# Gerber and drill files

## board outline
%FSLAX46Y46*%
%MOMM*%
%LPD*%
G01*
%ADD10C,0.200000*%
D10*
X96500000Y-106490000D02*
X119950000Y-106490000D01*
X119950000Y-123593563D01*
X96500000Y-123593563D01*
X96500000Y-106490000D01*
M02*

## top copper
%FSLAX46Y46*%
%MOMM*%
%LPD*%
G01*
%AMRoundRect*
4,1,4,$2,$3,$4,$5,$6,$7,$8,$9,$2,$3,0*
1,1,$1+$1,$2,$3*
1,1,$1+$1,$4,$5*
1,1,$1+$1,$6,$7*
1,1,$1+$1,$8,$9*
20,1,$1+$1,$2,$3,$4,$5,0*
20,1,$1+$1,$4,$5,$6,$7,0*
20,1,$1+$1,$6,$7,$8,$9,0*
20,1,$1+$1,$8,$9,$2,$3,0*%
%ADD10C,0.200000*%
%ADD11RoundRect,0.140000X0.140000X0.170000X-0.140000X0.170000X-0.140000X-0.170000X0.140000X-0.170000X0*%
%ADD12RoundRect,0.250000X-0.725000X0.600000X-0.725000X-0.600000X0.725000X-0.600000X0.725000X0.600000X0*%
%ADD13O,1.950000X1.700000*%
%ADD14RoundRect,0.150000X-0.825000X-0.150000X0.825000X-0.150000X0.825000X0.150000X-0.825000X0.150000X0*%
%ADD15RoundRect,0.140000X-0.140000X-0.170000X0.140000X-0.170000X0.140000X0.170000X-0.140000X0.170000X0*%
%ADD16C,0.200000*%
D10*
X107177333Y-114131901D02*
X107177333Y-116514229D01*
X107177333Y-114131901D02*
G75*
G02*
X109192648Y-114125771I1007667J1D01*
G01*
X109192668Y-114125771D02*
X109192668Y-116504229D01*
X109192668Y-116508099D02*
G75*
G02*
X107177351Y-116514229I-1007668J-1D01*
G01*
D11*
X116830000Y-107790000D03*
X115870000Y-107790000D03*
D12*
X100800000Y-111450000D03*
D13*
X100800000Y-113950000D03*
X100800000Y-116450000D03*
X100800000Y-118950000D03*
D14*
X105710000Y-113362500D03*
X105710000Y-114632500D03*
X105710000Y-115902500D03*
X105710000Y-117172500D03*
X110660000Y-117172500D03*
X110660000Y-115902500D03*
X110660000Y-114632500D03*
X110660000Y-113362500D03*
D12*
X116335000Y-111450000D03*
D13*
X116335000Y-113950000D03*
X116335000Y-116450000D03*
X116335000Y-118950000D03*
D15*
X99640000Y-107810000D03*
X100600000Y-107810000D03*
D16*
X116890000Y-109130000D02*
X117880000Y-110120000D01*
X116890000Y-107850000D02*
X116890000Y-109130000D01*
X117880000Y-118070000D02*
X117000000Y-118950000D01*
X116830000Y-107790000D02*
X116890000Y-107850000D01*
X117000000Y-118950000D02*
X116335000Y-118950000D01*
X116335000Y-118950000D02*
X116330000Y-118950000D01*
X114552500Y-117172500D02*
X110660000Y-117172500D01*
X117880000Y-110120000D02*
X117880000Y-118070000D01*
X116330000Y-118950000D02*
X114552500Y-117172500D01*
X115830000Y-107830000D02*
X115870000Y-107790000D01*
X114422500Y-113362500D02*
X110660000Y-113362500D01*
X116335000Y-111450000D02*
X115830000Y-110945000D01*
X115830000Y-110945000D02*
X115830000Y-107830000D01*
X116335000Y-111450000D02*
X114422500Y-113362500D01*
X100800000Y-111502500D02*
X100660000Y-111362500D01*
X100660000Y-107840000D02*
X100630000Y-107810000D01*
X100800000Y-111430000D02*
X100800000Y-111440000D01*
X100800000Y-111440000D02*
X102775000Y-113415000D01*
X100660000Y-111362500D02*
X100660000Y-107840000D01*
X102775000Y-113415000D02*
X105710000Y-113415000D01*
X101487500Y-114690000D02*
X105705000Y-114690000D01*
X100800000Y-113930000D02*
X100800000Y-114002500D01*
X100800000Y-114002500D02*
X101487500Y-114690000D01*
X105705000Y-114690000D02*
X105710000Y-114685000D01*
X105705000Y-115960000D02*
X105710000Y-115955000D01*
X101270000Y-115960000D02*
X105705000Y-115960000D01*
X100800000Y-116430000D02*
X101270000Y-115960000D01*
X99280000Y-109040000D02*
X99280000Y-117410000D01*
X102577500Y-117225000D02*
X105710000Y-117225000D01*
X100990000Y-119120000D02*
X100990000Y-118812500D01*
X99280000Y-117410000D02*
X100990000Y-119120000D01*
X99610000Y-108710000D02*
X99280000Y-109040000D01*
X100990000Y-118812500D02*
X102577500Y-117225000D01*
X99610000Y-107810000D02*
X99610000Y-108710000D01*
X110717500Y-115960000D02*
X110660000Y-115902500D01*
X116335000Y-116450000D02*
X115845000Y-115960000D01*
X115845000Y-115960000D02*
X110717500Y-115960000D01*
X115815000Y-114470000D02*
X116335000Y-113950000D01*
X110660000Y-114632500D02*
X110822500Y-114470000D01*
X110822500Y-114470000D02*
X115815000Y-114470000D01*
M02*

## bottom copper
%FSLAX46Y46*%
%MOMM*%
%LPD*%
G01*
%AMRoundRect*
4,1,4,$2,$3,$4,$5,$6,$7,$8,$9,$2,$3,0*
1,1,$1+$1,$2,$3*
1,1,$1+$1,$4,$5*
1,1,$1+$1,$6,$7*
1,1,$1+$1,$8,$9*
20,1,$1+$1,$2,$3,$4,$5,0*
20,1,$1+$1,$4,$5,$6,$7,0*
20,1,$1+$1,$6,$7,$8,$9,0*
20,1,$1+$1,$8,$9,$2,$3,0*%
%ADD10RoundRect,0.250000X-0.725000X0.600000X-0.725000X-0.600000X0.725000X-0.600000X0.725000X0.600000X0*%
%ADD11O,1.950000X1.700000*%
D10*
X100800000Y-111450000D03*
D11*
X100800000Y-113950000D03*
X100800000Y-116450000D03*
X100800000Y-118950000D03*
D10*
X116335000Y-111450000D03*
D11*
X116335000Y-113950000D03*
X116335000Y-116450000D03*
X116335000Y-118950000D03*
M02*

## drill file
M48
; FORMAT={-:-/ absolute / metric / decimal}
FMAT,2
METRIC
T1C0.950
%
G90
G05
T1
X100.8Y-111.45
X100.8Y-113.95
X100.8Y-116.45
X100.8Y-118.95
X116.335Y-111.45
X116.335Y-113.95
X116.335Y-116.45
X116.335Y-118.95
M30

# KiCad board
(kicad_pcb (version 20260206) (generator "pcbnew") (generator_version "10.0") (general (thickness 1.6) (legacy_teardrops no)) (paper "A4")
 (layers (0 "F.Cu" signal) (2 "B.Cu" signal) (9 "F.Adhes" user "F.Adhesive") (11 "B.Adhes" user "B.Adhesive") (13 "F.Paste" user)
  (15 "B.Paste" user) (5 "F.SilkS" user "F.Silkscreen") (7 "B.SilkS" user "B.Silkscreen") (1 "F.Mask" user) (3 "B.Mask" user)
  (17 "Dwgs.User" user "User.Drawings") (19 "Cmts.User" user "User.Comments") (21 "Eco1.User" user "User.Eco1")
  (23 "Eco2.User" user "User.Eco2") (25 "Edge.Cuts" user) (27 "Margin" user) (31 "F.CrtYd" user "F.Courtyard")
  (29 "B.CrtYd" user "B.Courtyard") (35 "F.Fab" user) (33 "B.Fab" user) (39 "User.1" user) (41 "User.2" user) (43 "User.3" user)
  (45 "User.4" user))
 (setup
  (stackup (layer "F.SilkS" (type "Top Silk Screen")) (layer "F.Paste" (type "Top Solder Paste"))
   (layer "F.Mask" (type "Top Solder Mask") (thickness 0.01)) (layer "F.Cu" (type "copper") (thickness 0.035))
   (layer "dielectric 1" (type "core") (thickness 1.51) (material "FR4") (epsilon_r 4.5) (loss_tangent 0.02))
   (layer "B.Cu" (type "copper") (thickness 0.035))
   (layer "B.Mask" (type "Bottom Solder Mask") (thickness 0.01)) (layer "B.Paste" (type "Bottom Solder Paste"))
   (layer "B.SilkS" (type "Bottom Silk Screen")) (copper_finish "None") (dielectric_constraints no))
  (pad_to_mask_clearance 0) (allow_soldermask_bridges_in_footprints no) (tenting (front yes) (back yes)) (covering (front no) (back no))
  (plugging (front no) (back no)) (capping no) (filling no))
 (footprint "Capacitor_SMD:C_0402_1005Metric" (layer "F.Cu") (at 116.35 107.79 180)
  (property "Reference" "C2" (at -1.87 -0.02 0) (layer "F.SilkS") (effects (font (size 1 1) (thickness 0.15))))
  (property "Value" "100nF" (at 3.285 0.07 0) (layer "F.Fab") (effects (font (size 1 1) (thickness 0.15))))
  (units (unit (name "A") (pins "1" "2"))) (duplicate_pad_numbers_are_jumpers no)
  (pad "1" smd roundrect (at -0.48 0 180) (size 0.56 0.62) (layers "F.Cu" "F.Mask" "F.Paste") (roundrect_rratio 0.25) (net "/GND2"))
  (pad "2" smd roundrect (at 0.48 0 180) (size 0.56 0.62) (layers "F.Cu" "F.Mask" "F.Paste") (roundrect_rratio 0.25) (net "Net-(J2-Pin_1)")))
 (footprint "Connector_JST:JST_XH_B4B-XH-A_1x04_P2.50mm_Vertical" (layer "F.Cu") (at 100.8 111.45 -90)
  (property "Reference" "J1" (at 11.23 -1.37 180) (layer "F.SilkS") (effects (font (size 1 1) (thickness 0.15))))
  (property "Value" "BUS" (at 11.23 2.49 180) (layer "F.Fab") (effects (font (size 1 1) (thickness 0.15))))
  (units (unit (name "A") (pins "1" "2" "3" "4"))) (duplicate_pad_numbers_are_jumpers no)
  (pad "1" thru_hole roundrect (at 0 0 270) (size 1.7 1.95) (drill 0.95) (layers "*.Cu" "*.Mask") (remove_unused_layers no)
   (roundrect_rratio 0.147059) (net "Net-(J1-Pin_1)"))
  (pad "2" thru_hole oval (at 2.5 0 270) (size 1.7 1.95) (drill 0.95) (layers "*.Cu" "*.Mask") (remove_unused_layers no)
   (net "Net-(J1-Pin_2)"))
  (pad "3" thru_hole oval (at 5 0 270) (size 1.7 1.95) (drill 0.95) (layers "*.Cu" "*.Mask") (remove_unused_layers no)
   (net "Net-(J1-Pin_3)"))
  (pad "4" thru_hole oval (at 7.5 0 270) (size 1.7 1.95) (drill 0.95) (layers "*.Cu" "*.Mask") (remove_unused_layers no) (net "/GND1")))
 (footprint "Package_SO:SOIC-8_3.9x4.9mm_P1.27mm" (layer "F.Cu") (at 108.185 115.2675)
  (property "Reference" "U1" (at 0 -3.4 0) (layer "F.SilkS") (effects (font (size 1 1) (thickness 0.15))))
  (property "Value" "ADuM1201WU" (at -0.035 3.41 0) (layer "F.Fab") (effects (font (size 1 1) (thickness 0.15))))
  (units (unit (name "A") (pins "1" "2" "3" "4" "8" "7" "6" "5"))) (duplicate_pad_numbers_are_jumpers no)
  (pad "1" smd roundrect (at -2.475 -1.905) (size 1.95 0.6) (layers "F.Cu" "F.Mask" "F.Paste") (roundrect_rratio 0.25)
   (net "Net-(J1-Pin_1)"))
  (pad "2" smd roundrect (at -2.475 -0.635) (size 1.95 0.6) (layers "F.Cu" "F.Mask" "F.Paste") (roundrect_rratio 0.25)
   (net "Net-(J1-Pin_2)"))
  (pad "3" smd roundrect (at -2.475 0.635) (size 1.95 0.6) (layers "F.Cu" "F.Mask" "F.Paste") (roundrect_rratio 0.25) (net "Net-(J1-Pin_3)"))
  (pad "4" smd roundrect (at -2.475 1.905) (size 1.95 0.6) (layers "F.Cu" "F.Mask" "F.Paste") (roundrect_rratio 0.25) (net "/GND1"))
  (pad "5" smd roundrect (at 2.475 1.905) (size 1.95 0.6) (layers "F.Cu" "F.Mask" "F.Paste") (roundrect_rratio 0.25) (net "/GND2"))
  (pad "6" smd roundrect (at 2.475 0.635) (size 1.95 0.6) (layers "F.Cu" "F.Mask" "F.Paste") (roundrect_rratio 0.25) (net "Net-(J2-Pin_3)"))
  (pad "7" smd roundrect (at 2.475 -0.635) (size 1.95 0.6) (layers "F.Cu" "F.Mask" "F.Paste") (roundrect_rratio 0.25) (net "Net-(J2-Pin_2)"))
  (pad "8" smd roundrect (at 2.475 -1.905) (size 1.95 0.6) (layers "F.Cu" "F.Mask" "F.Paste") (roundrect_rratio 0.25) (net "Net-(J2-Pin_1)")))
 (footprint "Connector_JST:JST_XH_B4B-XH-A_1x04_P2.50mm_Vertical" (layer "F.Cu") (at 116.335 111.45 -90)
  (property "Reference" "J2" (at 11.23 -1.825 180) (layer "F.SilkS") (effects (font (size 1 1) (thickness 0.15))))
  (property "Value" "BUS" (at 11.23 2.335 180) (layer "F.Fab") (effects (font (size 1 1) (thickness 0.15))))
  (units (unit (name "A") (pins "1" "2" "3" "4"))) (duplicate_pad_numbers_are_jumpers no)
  (pad "1" thru_hole roundrect (at 0 0 270) (size 1.7 1.95) (drill 0.95) (layers "*.Cu" "*.Mask") (remove_unused_layers no)
   (roundrect_rratio 0.147059) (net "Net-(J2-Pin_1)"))
  (pad "2" thru_hole oval (at 2.5 0 270) (size 1.7 1.95) (drill 0.95) (layers "*.Cu" "*.Mask") (remove_unused_layers no)
   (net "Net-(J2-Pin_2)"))
  (pad "3" thru_hole oval (at 5 0 270) (size 1.7 1.95) (drill 0.95) (layers "*.Cu" "*.Mask") (remove_unused_layers no)
   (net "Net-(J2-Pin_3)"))
  (pad "4" thru_hole oval (at 7.5 0 270) (size 1.7 1.95) (drill 0.95) (layers "*.Cu" "*.Mask") (remove_unused_layers no) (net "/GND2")))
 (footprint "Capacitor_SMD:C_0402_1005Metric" (layer "F.Cu") (at 100.12 107.81)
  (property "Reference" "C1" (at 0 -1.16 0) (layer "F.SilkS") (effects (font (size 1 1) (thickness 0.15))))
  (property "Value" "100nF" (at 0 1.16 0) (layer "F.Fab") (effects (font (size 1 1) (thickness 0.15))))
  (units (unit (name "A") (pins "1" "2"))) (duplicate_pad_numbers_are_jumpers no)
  (pad "1" smd roundrect (at -0.48 0) (size 0.56 0.62) (layers "F.Cu" "F.Mask" "F.Paste") (roundrect_rratio 0.25) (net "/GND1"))
  (pad "2" smd roundrect (at 0.48 0) (size 0.56 0.62) (layers "F.Cu" "F.Mask" "F.Paste") (roundrect_rratio 0.25) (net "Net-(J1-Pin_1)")))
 (gr_line (start 107.177333 114.131901) (end 107.177333 116.514229) (stroke (width 0.2) (type default)) (layer "F.Cu"))
 (gr_arc (start 107.177333 114.131901) (mid 108.181945 113.124229) (end 109.192668 114.125771) (stroke (width 0.2) (type default))
  (layer "F.Cu"))
 (gr_line (start 109.192668 114.125771) (end 109.192668 116.504229) (stroke (width 0.2) (type default)) (layer "F.Cu"))
 (gr_arc (start 109.192668 116.508099) (mid 108.188056 117.515771) (end 107.177333 116.514229) (stroke (width 0.2) (type default))
  (layer "F.Cu"))
 (gr_rect (start 96.5 106.49) (end 119.95 123.593563) (stroke (width 0.2) (type solid)) (fill no) (layer "Edge.Cuts"))
 (segment (start 116.89 109.13) (end 117.88 110.12) (width 0.2) (layer "F.Cu") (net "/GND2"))
 (segment (start 116.89 107.85) (end 116.89 109.13) (width 0.2) (layer "F.Cu") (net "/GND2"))
 (segment (start 117.88 118.07) (end 117 118.95) (width 0.2) (layer "F.Cu") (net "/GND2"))
 (segment (start 116.83 107.79) (end 116.89 107.85) (width 0.2) (layer "F.Cu") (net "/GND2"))
 (segment (start 117 118.95) (end 116.335 118.95) (width 0.2) (layer "F.Cu") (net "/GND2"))
 (segment (start 116.335 118.95) (end 116.33 118.95) (width 0.2) (layer "F.Cu") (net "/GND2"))
 (segment (start 114.5525 117.1725) (end 110.66 117.1725) (width 0.2) (layer "F.Cu") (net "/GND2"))
 (segment (start 117.88 110.12) (end 117.88 118.07) (width 0.2) (layer "F.Cu") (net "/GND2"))
 (segment (start 116.33 118.95) (end 114.5525 117.1725) (width 0.2) (layer "F.Cu") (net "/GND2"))
 (segment (start 115.83 107.83) (end 115.87 107.79) (width 0.2) (layer "F.Cu") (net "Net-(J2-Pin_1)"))
 (segment (start 114.4225 113.3625) (end 110.66 113.3625) (width 0.2) (layer "F.Cu") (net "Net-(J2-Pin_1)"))
 (segment (start 116.335 111.45) (end 115.83 110.945) (width 0.2) (layer "F.Cu") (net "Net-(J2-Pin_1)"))
 (segment (start 115.83 110.945) (end 115.83 107.83) (width 0.2) (layer "F.Cu") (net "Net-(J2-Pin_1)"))
 (segment (start 116.335 111.45) (end 114.4225 113.3625) (width 0.2) (layer "F.Cu") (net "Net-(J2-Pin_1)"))
 (segment (start 100.8 111.5025) (end 100.66 111.3625) (width 0.2) (layer "F.Cu") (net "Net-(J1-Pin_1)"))
 (segment (start 100.66 107.84) (end 100.63 107.81) (width 0.2) (layer "F.Cu") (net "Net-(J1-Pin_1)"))
 (segment (start 100.8 111.43) (end 100.8 111.44) (width 0.2) (layer "F.Cu") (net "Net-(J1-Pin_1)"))
 (segment (start 100.8 111.44) (end 102.775 113.415) (width 0.2) (layer "F.Cu") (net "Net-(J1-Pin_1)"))
 (segment (start 100.66 111.3625) (end 100.66 107.84) (width 0.2) (layer "F.Cu") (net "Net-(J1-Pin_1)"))
 (segment (start 102.775 113.415) (end 105.71 113.415) (width 0.2) (layer "F.Cu") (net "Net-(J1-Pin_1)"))
 (segment (start 101.4875 114.69) (end 105.705 114.69) (width 0.2) (layer "F.Cu") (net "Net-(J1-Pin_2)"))
 (segment (start 100.8 113.93) (end 100.8 114.0025) (width 0.2) (layer "F.Cu") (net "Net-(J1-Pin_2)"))
 (segment (start 100.8 114.0025) (end 101.4875 114.69) (width 0.2) (layer "F.Cu") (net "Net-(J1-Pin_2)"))
 (segment (start 105.705 114.69) (end 105.71 114.685) (width 0.2) (layer "F.Cu") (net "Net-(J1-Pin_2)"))
 (segment (start 105.705 115.96) (end 105.71 115.955) (width 0.2) (layer "F.Cu") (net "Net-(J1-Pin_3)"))
 (segment (start 101.27 115.96) (end 105.705 115.96) (width 0.2) (layer "F.Cu") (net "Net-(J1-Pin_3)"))
 (segment (start 100.8 116.43) (end 101.27 115.96) (width 0.2) (layer "F.Cu") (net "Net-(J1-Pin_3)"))
 (segment (start 99.28 109.04) (end 99.28 117.41) (width 0.2) (layer "F.Cu") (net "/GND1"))
 (segment (start 102.5775 117.225) (end 105.71 117.225) (width 0.2) (layer "F.Cu") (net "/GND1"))
 (segment (start 100.99 119.12) (end 100.99 118.8125) (width 0.2) (layer "F.Cu") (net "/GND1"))
 (segment (start 99.28 117.41) (end 100.99 119.12) (width 0.2) (layer "F.Cu") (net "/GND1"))
 (segment (start 99.61 108.71) (end 99.28 109.04) (width 0.2) (layer "F.Cu") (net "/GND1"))
 (segment (start 100.99 118.8125) (end 102.5775 117.225) (width 0.2) (layer "F.Cu") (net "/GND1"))
 (segment (start 99.61 107.81) (end 99.61 108.71) (width 0.2) (layer "F.Cu") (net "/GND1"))
 (segment (start 110.7175 115.96) (end 110.66 115.9025) (width 0.2) (layer "F.Cu") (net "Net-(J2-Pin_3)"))
 (segment (start 116.335 116.45) (end 115.845 115.96) (width 0.2) (layer "F.Cu") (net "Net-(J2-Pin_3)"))
 (segment (start 115.845 115.96) (end 110.7175 115.96) (width 0.2) (layer "F.Cu") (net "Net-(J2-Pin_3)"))
 (segment (start 115.815 114.47) (end 116.335 113.95) (width 0.2) (layer "F.Cu") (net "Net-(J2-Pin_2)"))
 (segment (start 110.66 114.6325) (end 110.8225 114.47) (width 0.2) (layer "F.Cu") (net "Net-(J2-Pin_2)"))
 (segment (start 110.8225 114.47) (end 115.815 114.47) (width 0.2) (layer "F.Cu") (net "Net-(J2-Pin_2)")))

